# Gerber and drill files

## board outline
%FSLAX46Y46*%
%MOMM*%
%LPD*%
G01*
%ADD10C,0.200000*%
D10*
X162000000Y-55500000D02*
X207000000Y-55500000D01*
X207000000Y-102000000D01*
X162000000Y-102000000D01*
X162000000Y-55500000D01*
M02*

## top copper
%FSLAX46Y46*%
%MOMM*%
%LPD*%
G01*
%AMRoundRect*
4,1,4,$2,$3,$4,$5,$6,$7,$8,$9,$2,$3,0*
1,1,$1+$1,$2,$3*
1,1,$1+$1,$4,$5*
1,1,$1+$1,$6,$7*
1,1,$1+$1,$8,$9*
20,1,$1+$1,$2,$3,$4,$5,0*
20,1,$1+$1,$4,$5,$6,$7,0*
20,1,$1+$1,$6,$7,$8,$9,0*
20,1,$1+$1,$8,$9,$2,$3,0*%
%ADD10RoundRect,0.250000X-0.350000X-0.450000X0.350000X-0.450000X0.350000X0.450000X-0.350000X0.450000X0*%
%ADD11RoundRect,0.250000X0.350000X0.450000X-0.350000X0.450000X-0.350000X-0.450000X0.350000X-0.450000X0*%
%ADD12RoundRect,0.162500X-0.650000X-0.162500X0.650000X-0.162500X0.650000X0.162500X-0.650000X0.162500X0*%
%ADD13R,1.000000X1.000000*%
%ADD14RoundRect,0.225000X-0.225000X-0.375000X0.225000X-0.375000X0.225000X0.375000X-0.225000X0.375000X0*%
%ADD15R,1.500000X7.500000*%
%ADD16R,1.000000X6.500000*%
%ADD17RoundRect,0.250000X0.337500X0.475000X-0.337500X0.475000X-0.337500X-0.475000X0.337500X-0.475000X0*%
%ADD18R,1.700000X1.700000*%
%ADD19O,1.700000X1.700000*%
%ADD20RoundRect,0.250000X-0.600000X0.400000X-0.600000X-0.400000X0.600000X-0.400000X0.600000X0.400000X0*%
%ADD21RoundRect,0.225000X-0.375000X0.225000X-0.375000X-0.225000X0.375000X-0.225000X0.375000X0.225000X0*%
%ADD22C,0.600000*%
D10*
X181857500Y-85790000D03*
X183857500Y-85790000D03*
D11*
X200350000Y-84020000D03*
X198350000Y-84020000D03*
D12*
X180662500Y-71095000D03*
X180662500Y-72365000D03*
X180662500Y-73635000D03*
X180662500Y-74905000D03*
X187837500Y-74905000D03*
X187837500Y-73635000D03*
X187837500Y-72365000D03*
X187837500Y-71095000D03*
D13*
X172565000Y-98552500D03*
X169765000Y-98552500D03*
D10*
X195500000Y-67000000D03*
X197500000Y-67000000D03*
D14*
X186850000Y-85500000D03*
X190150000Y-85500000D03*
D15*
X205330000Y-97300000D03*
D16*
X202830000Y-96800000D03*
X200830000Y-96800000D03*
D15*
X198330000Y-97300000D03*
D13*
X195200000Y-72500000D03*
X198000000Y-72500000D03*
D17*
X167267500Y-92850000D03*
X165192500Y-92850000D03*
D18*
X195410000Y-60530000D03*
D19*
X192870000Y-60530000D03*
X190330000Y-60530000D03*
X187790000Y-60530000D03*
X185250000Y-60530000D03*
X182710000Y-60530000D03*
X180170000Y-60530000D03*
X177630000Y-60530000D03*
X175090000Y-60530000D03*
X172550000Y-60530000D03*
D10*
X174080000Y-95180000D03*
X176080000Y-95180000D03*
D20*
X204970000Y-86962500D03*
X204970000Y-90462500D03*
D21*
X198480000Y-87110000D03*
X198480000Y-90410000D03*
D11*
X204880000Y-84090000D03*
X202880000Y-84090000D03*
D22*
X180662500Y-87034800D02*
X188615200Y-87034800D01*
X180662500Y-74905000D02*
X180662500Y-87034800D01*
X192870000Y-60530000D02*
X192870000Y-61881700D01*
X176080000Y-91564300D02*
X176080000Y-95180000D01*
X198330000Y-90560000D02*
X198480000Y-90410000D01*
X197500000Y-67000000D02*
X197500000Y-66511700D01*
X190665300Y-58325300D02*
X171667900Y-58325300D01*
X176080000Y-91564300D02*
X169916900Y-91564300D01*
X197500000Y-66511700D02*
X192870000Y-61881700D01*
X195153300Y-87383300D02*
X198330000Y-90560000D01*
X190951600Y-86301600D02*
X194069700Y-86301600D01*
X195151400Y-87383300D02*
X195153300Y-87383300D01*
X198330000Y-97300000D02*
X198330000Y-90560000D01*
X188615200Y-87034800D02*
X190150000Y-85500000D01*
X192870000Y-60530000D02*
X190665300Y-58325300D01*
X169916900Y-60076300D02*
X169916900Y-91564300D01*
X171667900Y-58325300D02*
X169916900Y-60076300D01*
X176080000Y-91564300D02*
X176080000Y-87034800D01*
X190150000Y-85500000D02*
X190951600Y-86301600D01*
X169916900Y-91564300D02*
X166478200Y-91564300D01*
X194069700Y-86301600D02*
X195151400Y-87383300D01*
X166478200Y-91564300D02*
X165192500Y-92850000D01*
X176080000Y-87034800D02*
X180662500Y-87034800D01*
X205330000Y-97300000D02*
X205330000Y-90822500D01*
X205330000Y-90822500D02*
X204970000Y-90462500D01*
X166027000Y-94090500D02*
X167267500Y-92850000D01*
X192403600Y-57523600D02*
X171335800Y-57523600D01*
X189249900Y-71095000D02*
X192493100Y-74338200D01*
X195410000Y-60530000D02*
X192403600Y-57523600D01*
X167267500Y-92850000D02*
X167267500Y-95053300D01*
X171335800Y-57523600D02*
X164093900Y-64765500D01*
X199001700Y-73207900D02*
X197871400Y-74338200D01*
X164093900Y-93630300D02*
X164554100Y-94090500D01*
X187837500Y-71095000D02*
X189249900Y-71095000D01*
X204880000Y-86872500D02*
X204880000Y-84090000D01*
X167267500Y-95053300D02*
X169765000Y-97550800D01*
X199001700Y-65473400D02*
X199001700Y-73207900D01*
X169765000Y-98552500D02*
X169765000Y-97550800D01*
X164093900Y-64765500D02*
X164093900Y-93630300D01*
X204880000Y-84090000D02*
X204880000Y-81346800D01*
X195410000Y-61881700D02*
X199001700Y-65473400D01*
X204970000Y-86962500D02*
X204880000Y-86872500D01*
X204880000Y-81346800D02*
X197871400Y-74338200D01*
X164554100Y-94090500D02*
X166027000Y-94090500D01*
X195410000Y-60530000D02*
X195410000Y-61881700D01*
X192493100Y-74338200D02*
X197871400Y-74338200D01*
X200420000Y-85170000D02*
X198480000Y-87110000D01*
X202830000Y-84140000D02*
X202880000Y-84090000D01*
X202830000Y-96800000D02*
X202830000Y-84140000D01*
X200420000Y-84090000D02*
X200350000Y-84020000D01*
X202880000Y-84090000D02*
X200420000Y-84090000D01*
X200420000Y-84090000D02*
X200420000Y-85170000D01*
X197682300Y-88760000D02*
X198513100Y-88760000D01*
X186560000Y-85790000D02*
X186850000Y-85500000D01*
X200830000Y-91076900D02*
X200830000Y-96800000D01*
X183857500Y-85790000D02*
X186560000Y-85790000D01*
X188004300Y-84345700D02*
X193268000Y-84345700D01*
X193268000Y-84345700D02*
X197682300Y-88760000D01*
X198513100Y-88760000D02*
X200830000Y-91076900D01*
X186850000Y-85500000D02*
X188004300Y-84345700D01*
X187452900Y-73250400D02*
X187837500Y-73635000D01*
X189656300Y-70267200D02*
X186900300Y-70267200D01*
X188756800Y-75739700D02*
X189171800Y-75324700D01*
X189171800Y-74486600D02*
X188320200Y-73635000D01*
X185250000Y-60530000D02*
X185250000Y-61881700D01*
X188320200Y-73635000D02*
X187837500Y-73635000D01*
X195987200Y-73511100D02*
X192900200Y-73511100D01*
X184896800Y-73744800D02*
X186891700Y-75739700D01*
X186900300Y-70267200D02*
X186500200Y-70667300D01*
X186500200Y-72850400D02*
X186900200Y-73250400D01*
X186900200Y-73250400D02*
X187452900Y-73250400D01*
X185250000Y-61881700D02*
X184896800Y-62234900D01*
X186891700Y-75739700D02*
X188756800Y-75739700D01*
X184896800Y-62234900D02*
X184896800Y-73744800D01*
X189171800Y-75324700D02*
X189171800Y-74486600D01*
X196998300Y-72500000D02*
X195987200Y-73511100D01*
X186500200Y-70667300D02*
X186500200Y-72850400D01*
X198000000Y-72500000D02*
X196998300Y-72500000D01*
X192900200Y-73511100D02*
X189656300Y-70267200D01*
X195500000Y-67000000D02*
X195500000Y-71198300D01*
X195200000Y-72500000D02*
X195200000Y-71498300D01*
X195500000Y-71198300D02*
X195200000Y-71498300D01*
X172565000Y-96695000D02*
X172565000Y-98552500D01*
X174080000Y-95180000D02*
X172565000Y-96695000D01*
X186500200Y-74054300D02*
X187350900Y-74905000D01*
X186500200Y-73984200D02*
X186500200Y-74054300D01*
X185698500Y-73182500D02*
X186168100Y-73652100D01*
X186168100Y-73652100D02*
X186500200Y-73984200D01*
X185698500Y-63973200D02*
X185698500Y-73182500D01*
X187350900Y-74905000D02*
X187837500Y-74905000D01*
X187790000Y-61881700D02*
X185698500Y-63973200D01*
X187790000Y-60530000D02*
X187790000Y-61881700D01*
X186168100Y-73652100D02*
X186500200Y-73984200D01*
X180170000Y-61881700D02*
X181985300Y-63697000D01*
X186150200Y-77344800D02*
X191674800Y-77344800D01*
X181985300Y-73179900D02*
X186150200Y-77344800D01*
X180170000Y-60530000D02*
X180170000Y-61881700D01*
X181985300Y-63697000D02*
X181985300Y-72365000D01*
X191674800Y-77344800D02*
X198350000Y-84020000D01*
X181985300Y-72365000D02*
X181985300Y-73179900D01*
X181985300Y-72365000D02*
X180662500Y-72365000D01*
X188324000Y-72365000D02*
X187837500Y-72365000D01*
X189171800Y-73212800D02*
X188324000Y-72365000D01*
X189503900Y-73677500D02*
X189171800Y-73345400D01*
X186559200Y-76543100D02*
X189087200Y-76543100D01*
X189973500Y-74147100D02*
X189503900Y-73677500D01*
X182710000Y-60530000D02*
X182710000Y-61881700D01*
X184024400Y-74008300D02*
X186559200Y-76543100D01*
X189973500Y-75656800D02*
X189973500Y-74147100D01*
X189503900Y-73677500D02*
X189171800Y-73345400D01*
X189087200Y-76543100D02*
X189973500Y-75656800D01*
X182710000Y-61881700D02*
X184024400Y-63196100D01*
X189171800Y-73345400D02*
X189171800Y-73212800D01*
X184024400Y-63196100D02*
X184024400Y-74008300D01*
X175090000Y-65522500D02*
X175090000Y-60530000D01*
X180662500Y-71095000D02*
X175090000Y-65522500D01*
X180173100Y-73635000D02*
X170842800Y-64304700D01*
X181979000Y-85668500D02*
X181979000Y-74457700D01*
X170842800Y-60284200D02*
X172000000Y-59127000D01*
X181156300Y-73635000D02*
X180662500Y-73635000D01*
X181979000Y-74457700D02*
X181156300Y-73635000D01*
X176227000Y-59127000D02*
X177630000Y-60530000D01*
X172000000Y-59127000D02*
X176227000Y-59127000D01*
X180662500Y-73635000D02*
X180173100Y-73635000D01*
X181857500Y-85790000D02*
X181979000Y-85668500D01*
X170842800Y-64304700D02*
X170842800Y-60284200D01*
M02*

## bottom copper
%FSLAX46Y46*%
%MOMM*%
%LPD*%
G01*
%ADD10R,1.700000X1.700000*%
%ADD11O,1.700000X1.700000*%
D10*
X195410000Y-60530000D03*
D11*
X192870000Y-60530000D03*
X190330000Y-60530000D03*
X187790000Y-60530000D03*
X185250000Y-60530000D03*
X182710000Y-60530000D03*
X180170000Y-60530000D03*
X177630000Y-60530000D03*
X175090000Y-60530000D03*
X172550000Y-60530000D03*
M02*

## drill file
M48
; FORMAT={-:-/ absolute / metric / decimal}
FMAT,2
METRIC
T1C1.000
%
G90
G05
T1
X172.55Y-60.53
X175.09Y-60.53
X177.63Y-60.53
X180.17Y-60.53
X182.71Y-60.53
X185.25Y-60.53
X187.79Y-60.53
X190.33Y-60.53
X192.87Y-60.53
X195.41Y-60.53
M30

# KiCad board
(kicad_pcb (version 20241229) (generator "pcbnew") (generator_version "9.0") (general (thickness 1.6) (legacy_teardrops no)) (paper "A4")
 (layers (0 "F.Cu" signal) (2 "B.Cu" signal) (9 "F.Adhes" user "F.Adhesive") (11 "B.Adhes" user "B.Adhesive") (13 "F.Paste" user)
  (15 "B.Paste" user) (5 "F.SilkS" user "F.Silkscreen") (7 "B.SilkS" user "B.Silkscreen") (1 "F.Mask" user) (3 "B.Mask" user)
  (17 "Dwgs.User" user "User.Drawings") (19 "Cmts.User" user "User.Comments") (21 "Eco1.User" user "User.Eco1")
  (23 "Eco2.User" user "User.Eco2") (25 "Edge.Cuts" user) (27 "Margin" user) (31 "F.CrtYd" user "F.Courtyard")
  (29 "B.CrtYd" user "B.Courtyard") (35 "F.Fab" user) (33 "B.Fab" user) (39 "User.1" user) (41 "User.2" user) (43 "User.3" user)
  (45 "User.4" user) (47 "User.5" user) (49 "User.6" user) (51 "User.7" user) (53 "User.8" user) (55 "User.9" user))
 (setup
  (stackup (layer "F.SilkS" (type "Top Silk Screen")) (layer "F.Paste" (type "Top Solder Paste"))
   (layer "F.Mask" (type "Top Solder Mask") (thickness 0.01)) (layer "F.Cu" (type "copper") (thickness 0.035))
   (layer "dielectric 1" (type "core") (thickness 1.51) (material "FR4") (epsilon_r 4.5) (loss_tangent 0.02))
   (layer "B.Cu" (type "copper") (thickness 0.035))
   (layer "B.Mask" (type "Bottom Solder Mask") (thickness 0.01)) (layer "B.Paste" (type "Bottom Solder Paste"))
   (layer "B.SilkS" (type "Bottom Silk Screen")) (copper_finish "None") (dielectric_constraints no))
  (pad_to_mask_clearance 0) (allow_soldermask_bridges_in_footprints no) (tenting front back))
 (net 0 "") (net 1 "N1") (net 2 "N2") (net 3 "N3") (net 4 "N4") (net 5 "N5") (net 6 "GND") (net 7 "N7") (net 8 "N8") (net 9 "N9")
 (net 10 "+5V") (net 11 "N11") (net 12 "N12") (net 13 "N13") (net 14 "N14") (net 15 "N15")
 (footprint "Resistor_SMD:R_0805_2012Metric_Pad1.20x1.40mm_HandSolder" (layer "F.Cu") (at 182.8575 85.79)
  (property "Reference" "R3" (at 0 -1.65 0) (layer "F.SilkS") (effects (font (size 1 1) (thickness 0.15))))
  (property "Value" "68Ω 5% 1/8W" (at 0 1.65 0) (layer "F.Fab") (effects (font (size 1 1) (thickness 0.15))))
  (pad "1" smd roundrect (at -1 0) (size 1.2 1.4) (layers "F.Cu" "F.Mask" "F.Paste") (roundrect_rratio 0.208333) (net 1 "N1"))
  (pad "2" smd roundrect (at 1 0) (size 1.2 1.4) (layers "F.Cu" "F.Mask" "F.Paste") (roundrect_rratio 0.208333) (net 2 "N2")))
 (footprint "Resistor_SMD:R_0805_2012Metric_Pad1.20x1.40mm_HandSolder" (layer "F.Cu") (at 199.35 84.02 180)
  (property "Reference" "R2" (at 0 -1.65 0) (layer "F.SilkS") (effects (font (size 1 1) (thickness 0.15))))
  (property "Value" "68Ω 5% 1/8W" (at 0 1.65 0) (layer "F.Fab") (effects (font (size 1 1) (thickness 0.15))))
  (pad "1" smd roundrect (at -1 0 180) (size 1.2 1.4) (layers "F.Cu" "F.Mask" "F.Paste") (roundrect_rratio 0.208333) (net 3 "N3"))
  (pad "2" smd roundrect (at 1 0 180) (size 1.2 1.4) (layers "F.Cu" "F.Mask" "F.Paste") (roundrect_rratio 0.208333) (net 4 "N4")))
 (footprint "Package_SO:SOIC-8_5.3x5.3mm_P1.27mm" (layer "F.Cu") (at 184.25 73)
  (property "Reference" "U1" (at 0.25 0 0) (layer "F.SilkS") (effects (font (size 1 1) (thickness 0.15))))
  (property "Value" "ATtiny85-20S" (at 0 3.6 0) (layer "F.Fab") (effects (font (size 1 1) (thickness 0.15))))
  (pad "1" smd roundrect (at -3.5875 -1.905) (size 1.625 0.65) (layers "F.Cu" "F.Mask" "F.Paste") (roundrect_rratio 0.25) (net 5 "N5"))
  (pad "2" smd roundrect (at -3.5875 -0.635) (size 1.625 0.65) (layers "F.Cu" "F.Mask" "F.Paste") (roundrect_rratio 0.25) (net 4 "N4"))
  (pad "3" smd roundrect (at -3.5875 0.635) (size 1.625 0.65) (layers "F.Cu" "F.Mask" "F.Paste") (roundrect_rratio 0.25) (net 1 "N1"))
  (pad "4" smd roundrect (at -3.5875 1.905) (size 1.625 0.65) (layers "F.Cu" "F.Mask" "F.Paste") (roundrect_rratio 0.25) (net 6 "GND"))
  (pad "5" smd roundrect (at 3.5875 1.905) (size 1.625 0.65) (layers "F.Cu" "F.Mask" "F.Paste") (roundrect_rratio 0.25) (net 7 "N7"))
  (pad "6" smd roundrect (at 3.5875 0.635) (size 1.625 0.65) (layers "F.Cu" "F.Mask" "F.Paste") (roundrect_rratio 0.25) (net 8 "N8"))
  (pad "7" smd roundrect (at 3.5875 -0.635) (size 1.625 0.65) (layers "F.Cu" "F.Mask" "F.Paste") (roundrect_rratio 0.25) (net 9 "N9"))
  (pad "8" smd roundrect (at 3.5875 -1.905) (size 1.625 0.65) (layers "F.Cu" "F.Mask" "F.Paste") (roundrect_rratio 0.25) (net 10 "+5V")))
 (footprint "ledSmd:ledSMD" (layer "F.Cu") (at 170.765 98.5525 180)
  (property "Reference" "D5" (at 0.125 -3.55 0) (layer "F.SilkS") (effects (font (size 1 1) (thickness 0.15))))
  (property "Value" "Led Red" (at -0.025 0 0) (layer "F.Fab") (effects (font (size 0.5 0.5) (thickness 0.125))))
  (pad "1" smd rect (at -1.8 0 180) (size 1 1) (layers "F.Cu" "F.Mask" "F.Paste") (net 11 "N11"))
  (pad "2" smd rect (at 1 0 180) (size 1 1) (layers "F.Cu" "F.Mask" "F.Paste") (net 10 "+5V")))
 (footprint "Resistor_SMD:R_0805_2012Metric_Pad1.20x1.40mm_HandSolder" (layer "F.Cu") (at 196.5 67)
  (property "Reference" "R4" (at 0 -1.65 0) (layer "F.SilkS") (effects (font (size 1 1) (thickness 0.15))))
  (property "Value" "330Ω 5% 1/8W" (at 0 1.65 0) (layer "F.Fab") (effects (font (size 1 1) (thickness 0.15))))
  (pad "1" smd roundrect (at -1 0) (size 1.2 1.4) (layers "F.Cu" "F.Mask" "F.Paste") (roundrect_rratio 0.208333) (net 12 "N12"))
  (pad "2" smd roundrect (at 1 0) (size 1.2 1.4) (layers "F.Cu" "F.Mask" "F.Paste") (roundrect_rratio 0.208333) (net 6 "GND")))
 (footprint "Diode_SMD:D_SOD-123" (layer "F.Cu") (at 188.5 85.5)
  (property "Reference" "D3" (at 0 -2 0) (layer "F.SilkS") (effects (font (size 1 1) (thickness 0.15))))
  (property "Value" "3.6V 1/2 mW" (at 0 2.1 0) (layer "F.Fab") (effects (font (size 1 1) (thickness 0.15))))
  (pad "1" smd roundrect (at -1.65 0) (size 0.9 1.2) (layers "F.Cu" "F.Mask" "F.Paste") (roundrect_rratio 0.25) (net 2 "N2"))
  (pad "2" smd roundrect (at 1.65 0) (size 0.9 1.2) (layers "F.Cu" "F.Mask" "F.Paste") (roundrect_rratio 0.25) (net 6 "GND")))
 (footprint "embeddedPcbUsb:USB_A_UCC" (layer "F.Cu") (at 201.83 97.1 90)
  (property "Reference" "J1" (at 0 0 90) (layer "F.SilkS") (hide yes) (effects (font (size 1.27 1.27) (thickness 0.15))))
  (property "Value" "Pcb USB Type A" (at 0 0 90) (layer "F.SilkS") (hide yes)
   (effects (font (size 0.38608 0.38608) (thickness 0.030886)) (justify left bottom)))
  (pad "1" smd rect (at -0.2 3.5 90) (size 7.5 1.5) (layers "F.Cu" "F.Mask" "F.Paste") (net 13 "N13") (solder_mask_margin 0.1016))
  (pad "2" smd rect (at 0.3 1 90) (size 6.5 1) (layers "F.Cu" "F.Mask" "F.Paste") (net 3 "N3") (solder_mask_margin 0.1016))
  (pad "3" smd rect (at 0.3 -1 90) (size 6.5 1) (layers "F.Cu" "F.Mask" "F.Paste") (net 2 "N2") (solder_mask_margin 0.1016))
  (pad "4" smd rect (at -0.2 -3.5 90) (size 7.5 1.5) (layers "F.Cu" "F.Mask" "F.Paste") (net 6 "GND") (solder_mask_margin 0.1016)))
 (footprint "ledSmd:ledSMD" (layer "F.Cu") (at 197 72.5)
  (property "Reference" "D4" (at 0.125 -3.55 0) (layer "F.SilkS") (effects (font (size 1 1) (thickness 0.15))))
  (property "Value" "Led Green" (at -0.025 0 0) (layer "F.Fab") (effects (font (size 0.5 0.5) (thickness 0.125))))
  (pad "1" smd rect (at -1.8 0) (size 1 1) (layers "F.Cu" "F.Mask" "F.Paste") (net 12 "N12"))
  (pad "2" smd rect (at 1 0) (size 1 1) (layers "F.Cu" "F.Mask" "F.Paste") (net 8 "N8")))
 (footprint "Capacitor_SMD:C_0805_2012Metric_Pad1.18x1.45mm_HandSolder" (layer "F.Cu") (at 166.23 92.85 180)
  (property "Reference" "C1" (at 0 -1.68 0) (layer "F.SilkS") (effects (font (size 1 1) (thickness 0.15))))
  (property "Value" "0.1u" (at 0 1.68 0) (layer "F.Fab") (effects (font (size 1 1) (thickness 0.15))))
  (pad "1" smd roundrect (at -1.0375 0 180) (size 1.175 1.45) (layers "F.Cu" "F.Mask" "F.Paste") (roundrect_rratio 0.212766) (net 10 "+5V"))
  (pad "2" smd roundrect (at 1.0375 0 180) (size 1.175 1.45) (layers "F.Cu" "F.Mask" "F.Paste") (roundrect_rratio 0.212766) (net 6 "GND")))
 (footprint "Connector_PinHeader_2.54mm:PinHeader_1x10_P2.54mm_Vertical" (layer "F.Cu") (at 195.41 60.53 -90)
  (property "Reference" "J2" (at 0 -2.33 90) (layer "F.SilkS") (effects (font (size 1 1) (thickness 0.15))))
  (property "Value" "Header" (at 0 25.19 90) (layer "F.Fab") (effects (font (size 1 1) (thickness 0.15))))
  (pad "1" thru_hole rect (at 0 0 270) (size 1.7 1.7) (drill 1) (layers "*.Cu" "*.Mask") (remove_unused_layers no) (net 10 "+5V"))
  (pad "2" thru_hole oval (at 0 2.54 270) (size 1.7 1.7) (drill 1) (layers "*.Cu" "*.Mask") (remove_unused_layers no) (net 6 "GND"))
  (pad "3" thru_hole oval (at 0 5.08 270) (size 1.7 1.7) (drill 1) (layers "*.Cu" "*.Mask") (remove_unused_layers no) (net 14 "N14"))
  (pad "4" thru_hole oval (at 0 7.62 270) (size 1.7 1.7) (drill 1) (layers "*.Cu" "*.Mask") (remove_unused_layers no) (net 7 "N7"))
  (pad "5" thru_hole oval (at 0 10.16 270) (size 1.7 1.7) (drill 1) (layers "*.Cu" "*.Mask") (remove_unused_layers no) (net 8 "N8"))
  (pad "6" thru_hole oval (at 0 12.7 270) (size 1.7 1.7) (drill 1) (layers "*.Cu" "*.Mask") (remove_unused_layers no) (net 9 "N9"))
  (pad "7" thru_hole oval (at 0 15.24 270) (size 1.7 1.7) (drill 1) (layers "*.Cu" "*.Mask") (remove_unused_layers no) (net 4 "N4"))
  (pad "8" thru_hole oval (at 0 17.78 270) (size 1.7 1.7) (drill 1) (layers "*.Cu" "*.Mask") (remove_unused_layers no) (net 1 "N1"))
  (pad "9" thru_hole oval (at 0 20.32 270) (size 1.7 1.7) (drill 1) (layers "*.Cu" "*.Mask") (remove_unused_layers no) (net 5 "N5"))
  (pad "10" thru_hole oval (at 0 22.86 270) (size 1.7 1.7) (drill 1) (layers "*.Cu" "*.Mask") (remove_unused_layers no) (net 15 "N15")))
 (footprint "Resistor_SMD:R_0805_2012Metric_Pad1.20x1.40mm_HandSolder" (layer "F.Cu") (at 175.08 95.18)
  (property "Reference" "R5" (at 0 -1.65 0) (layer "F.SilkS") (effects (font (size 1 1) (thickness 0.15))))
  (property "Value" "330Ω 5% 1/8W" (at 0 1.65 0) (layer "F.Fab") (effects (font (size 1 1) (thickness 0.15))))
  (pad "1" smd roundrect (at -1 0) (size 1.2 1.4) (layers "F.Cu" "F.Mask" "F.Paste") (roundrect_rratio 0.208333) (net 11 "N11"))
  (pad "2" smd roundrect (at 1 0) (size 1.2 1.4) (layers "F.Cu" "F.Mask" "F.Paste") (roundrect_rratio 0.208333) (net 6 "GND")))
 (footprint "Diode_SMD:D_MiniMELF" (layer "F.Cu") (at 204.97 88.7125 -90)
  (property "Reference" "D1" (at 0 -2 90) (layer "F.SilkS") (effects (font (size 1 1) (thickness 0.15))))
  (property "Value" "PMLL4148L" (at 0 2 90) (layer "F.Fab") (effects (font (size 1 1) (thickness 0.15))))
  (pad "1" smd roundrect (at -1.75 0 270) (size 1.3 1.7) (layers "F.Cu" "F.Mask" "F.Paste") (roundrect_rratio 0.1923076923) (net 10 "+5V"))
  (pad "2" smd roundrect (at 1.75 0 270) (size 1.3 1.7) (layers "F.Cu" "F.Mask" "F.Paste") (roundrect_rratio 0.1923076923) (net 13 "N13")))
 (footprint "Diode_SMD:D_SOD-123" (layer "F.Cu") (at 198.48 88.76 -90)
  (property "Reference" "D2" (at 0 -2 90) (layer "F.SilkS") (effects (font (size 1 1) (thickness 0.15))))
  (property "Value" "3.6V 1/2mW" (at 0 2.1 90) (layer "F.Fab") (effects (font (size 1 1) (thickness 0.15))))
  (pad "1" smd roundrect (at -1.65 0 270) (size 0.9 1.2) (layers "F.Cu" "F.Mask" "F.Paste") (roundrect_rratio 0.25) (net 3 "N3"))
  (pad "2" smd roundrect (at 1.65 0 270) (size 0.9 1.2) (layers "F.Cu" "F.Mask" "F.Paste") (roundrect_rratio 0.25) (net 6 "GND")))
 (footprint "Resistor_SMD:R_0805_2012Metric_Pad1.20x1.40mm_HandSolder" (layer "F.Cu") (at 203.88 84.09 180)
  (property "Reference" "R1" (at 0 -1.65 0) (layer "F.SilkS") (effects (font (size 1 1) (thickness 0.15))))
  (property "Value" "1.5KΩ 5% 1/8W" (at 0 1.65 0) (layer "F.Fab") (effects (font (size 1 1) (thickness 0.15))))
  (pad "1" smd roundrect (at -1 0 180) (size 1.2 1.4) (layers "F.Cu" "F.Mask" "F.Paste") (roundrect_rratio 0.208333) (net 10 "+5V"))
  (pad "2" smd roundrect (at 1 0 180) (size 1.2 1.4) (layers "F.Cu" "F.Mask" "F.Paste") (roundrect_rratio 0.208333) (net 3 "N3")))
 (gr_rect (start 162 55.5) (end 207 102) (stroke (width 0.2) (type solid)) (fill no) (layer "Edge.Cuts"))
 (segment (start 180.6625 87.0348) (end 188.6152 87.0348) (width 0.6) (layer "F.Cu") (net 6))
 (segment (start 180.6625 74.905) (end 180.6625 87.0348) (width 0.6) (layer "F.Cu") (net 6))
 (segment (start 192.87 60.53) (end 192.87 61.8817) (width 0.6) (layer "F.Cu") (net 6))
 (segment (start 176.08 91.5643) (end 176.08 95.18) (width 0.6) (layer "F.Cu") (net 6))
 (segment (start 198.33 90.56) (end 198.48 90.41) (width 0.6) (layer "F.Cu") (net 6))
 (segment (start 197.5 67) (end 197.5 66.5117) (width 0.6) (layer "F.Cu") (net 6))
 (segment (start 190.6653 58.3253) (end 171.6679 58.3253) (width 0.6) (layer "F.Cu") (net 6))
 (segment (start 176.08 91.5643) (end 169.9169 91.5643) (width 0.6) (layer "F.Cu") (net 6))
 (segment (start 197.5 66.5117) (end 192.87 61.8817) (width 0.6) (layer "F.Cu") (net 6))
 (segment (start 195.1533 87.3833) (end 198.33 90.56) (width 0.6) (layer "F.Cu") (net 6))
 (segment (start 190.9516 86.3016) (end 194.0697 86.3016) (width 0.6) (layer "F.Cu") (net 6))
 (segment (start 195.1514 87.3833) (end 195.1533 87.3833) (width 0.6) (layer "F.Cu") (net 6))
 (segment (start 198.33 97.3) (end 198.33 90.56) (width 0.6) (layer "F.Cu") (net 6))
 (segment (start 188.6152 87.0348) (end 190.15 85.5) (width 0.6) (layer "F.Cu") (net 6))
 (segment (start 192.87 60.53) (end 190.6653 58.3253) (width 0.6) (layer "F.Cu") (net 6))
 (segment (start 169.9169 60.0763) (end 169.9169 91.5643) (width 0.6) (layer "F.Cu") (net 6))
 (segment (start 171.6679 58.3253) (end 169.9169 60.0763) (width 0.6) (layer "F.Cu") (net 6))
 (segment (start 176.08 91.5643) (end 176.08 87.0348) (width 0.6) (layer "F.Cu") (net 6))
 (segment (start 190.15 85.5) (end 190.9516 86.3016) (width 0.6) (layer "F.Cu") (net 6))
 (segment (start 169.9169 91.5643) (end 166.4782 91.5643) (width 0.6) (layer "F.Cu") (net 6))
 (segment (start 194.0697 86.3016) (end 195.1514 87.3833) (width 0.6) (layer "F.Cu") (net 6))
 (segment (start 166.4782 91.5643) (end 165.1925 92.85) (width 0.6) (layer "F.Cu") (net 6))
 (segment (start 176.08 87.0348) (end 180.6625 87.0348) (width 0.6) (layer "F.Cu") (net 6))
 (segment (start 205.33 97.3) (end 205.33 90.8225) (width 0.6) (layer "F.Cu") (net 13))
 (segment (start 205.33 90.8225) (end 204.97 90.4625) (width 0.6) (layer "F.Cu") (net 13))
 (segment (start 166.027 94.0905) (end 167.2675 92.85) (width 0.6) (layer "F.Cu") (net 10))
 (segment (start 192.4036 57.5236) (end 171.3358 57.5236) (width 0.6) (layer "F.Cu") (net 10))
 (segment (start 189.2499 71.095) (end 192.4931 74.3382) (width 0.6) (layer "F.Cu") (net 10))
 (segment (start 195.41 60.53) (end 192.4036 57.5236) (width 0.6) (layer "F.Cu") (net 10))
 (segment (start 167.2675 92.85) (end 167.2675 95.0533) (width 0.6) (layer "F.Cu") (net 10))
 (segment (start 171.3358 57.5236) (end 164.0939 64.7655) (width 0.6) (layer "F.Cu") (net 10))
 (segment (start 199.0017 73.2079) (end 197.8714 74.3382) (width 0.6) (layer "F.Cu") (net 10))
 (segment (start 164.0939 93.6303) (end 164.5541 94.0905) (width 0.6) (layer "F.Cu") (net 10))
 (segment (start 187.8375 71.095) (end 189.2499 71.095) (width 0.6) (layer "F.Cu") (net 10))
 (segment (start 204.88 86.8725) (end 204.88 84.09) (width 0.6) (layer "F.Cu") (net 10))
 (segment (start 167.2675 95.0533) (end 169.765 97.5508) (width 0.6) (layer "F.Cu") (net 10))
 (segment (start 199.0017 65.4734) (end 199.0017 73.2079) (width 0.6) (layer "F.Cu") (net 10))
 (segment (start 169.765 98.5525) (end 169.765 97.5508) (width 0.6) (layer "F.Cu") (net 10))
 (segment (start 164.0939 64.7655) (end 164.0939 93.6303) (width 0.6) (layer "F.Cu") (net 10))
 (segment (start 204.88 84.09) (end 204.88 81.3468) (width 0.6) (layer "F.Cu") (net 10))
 (segment (start 195.41 61.8817) (end 199.0017 65.4734) (width 0.6) (layer "F.Cu") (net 10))
 (segment (start 204.97 86.9625) (end 204.88 86.8725) (width 0.6) (layer "F.Cu") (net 10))
 (segment (start 204.88 81.3468) (end 197.8714 74.3382) (width 0.6) (layer "F.Cu") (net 10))
 (segment (start 164.5541 94.0905) (end 166.027 94.0905) (width 0.6) (layer "F.Cu") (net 10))
 (segment (start 195.41 60.53) (end 195.41 61.8817) (width 0.6) (layer "F.Cu") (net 10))
 (segment (start 192.4931 74.3382) (end 197.8714 74.3382) (width 0.6) (layer "F.Cu") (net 10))
 (segment (start 200.42 85.17) (end 198.48 87.11) (width 0.6) (layer "F.Cu") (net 3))
 (segment (start 202.83 84.14) (end 202.88 84.09) (width 0.6) (layer "F.Cu") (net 3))
 (segment (start 202.83 96.8) (end 202.83 84.14) (width 0.6) (layer "F.Cu") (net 3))
 (segment (start 200.42 84.09) (end 200.35 84.02) (width 0.6) (layer "F.Cu") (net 3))
 (segment (start 202.88 84.09) (end 200.42 84.09) (width 0.6) (layer "F.Cu") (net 3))
 (segment (start 200.42 84.09) (end 200.42 85.17) (width 0.6) (layer "F.Cu") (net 3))
 (segment (start 197.6823 88.76) (end 198.5131 88.76) (width 0.6) (layer "F.Cu") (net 2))
 (segment (start 186.56 85.79) (end 186.85 85.5) (width 0.6) (layer "F.Cu") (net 2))
 (segment (start 200.83 91.0769) (end 200.83 96.8) (width 0.6) (layer "F.Cu") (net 2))
 (segment (start 183.8575 85.79) (end 186.56 85.79) (width 0.6) (layer "F.Cu") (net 2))
 (segment (start 188.0043 84.3457) (end 193.268 84.3457) (width 0.6) (layer "F.Cu") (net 2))
 (segment (start 193.268 84.3457) (end 197.6823 88.76) (width 0.6) (layer "F.Cu") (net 2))
 (segment (start 198.5131 88.76) (end 200.83 91.0769) (width 0.6) (layer "F.Cu") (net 2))
 (segment (start 186.85 85.5) (end 188.0043 84.3457) (width 0.6) (layer "F.Cu") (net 2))
 (segment (start 187.4529 73.2504) (end 187.8375 73.635) (width 0.6) (layer "F.Cu") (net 8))
 (segment (start 189.6563 70.2672) (end 186.9003 70.2672) (width 0.6) (layer "F.Cu") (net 8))
 (segment (start 188.7568 75.7397) (end 189.1718 75.3247) (width 0.6) (layer "F.Cu") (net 8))
 (segment (start 189.1718 74.4866) (end 188.3202 73.635) (width 0.6) (layer "F.Cu") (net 8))
 (segment (start 185.25 60.53) (end 185.25 61.8817) (width 0.6) (layer "F.Cu") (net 8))
 (segment (start 188.3202 73.635) (end 187.8375 73.635) (width 0.6) (layer "F.Cu") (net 8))
 (segment (start 195.9872 73.5111) (end 192.9002 73.5111) (width 0.6) (layer "F.Cu") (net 8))
 (segment (start 184.8968 73.7448) (end 186.8917 75.7397) (width 0.6) (layer "F.Cu") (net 8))
 (segment (start 186.9003 70.2672) (end 186.5002 70.6673) (width 0.6) (layer "F.Cu") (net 8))
 (segment (start 186.5002 72.8504) (end 186.9002 73.2504) (width 0.6) (layer "F.Cu") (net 8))
 (segment (start 186.9002 73.2504) (end 187.4529 73.2504) (width 0.6) (layer "F.Cu") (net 8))
 (segment (start 185.25 61.8817) (end 184.8968 62.2349) (width 0.6) (layer "F.Cu") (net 8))
 (segment (start 186.8917 75.7397) (end 188.7568 75.7397) (width 0.6) (layer "F.Cu") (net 8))
 (segment (start 184.8968 62.2349) (end 184.8968 73.7448) (width 0.6) (layer "F.Cu") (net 8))
 (segment (start 189.1718 75.3247) (end 189.1718 74.4866) (width 0.6) (layer "F.Cu") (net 8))
 (segment (start 196.9983 72.5) (end 195.9872 73.5111) (width 0.6) (layer "F.Cu") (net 8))
 (segment (start 186.5002 70.6673) (end 186.5002 72.8504) (width 0.6) (layer "F.Cu") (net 8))
 (segment (start 198 72.5) (end 196.9983 72.5) (width 0.6) (layer "F.Cu") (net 8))
 (segment (start 192.9002 73.5111) (end 189.6563 70.2672) (width 0.6) (layer "F.Cu") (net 8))
 (segment (start 195.5 67) (end 195.5 71.1983) (width 0.6) (layer "F.Cu") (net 12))
 (segment (start 195.2 72.5) (end 195.2 71.4983) (width 0.6) (layer "F.Cu") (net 12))
 (segment (start 195.5 71.1983) (end 195.2 71.4983) (width 0.6) (layer "F.Cu") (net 12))
 (segment (start 172.565 96.695) (end 172.565 98.5525) (width 0.6) (layer "F.Cu") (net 11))
 (segment (start 174.08 95.18) (end 172.565 96.695) (width 0.6) (layer "F.Cu") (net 11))
 (segment (start 186.5002 74.0543) (end 187.3509 74.905) (width 0.6) (layer "F.Cu") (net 7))
 (segment (start 186.5002 73.9842) (end 186.5002 74.0543) (width 0.6) (layer "F.Cu") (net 7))
 (segment (start 185.6985 73.1825) (end 186.1681 73.6521) (width 0.6) (layer "F.Cu") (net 7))
 (segment (start 186.1681 73.6521) (end 186.5002 73.9842) (width 0.6) (layer "F.Cu") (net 7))
 (segment (start 185.6985 63.9732) (end 185.6985 73.1825) (width 0.6) (layer "F.Cu") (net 7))
 (segment (start 187.3509 74.905) (end 187.8375 74.905) (width 0.6) (layer "F.Cu") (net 7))
 (segment (start 187.79 61.8817) (end 185.6985 63.9732) (width 0.6) (layer "F.Cu") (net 7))
 (segment (start 187.79 60.53) (end 187.79 61.8817) (width 0.6) (layer "F.Cu") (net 7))
 (segment (start 186.1681 73.6521) (end 186.5002 73.9842) (width 0.6) (layer "F.Cu") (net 7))
 (segment (start 180.17 61.8817) (end 181.9853 63.697) (width 0.6) (layer "F.Cu") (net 4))
 (segment (start 186.1502 77.3448) (end 191.6748 77.3448) (width 0.6) (layer "F.Cu") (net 4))
 (segment (start 181.9853 73.1799) (end 186.1502 77.3448) (width 0.6) (layer "F.Cu") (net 4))
 (segment (start 180.17 60.53) (end 180.17 61.8817) (width 0.6) (layer "F.Cu") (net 4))
 (segment (start 181.9853 63.697) (end 181.9853 72.365) (width 0.6) (layer "F.Cu") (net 4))
 (segment (start 191.6748 77.3448) (end 198.35 84.02) (width 0.6) (layer "F.Cu") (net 4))
 (segment (start 181.9853 72.365) (end 181.9853 73.1799) (width 0.6) (layer "F.Cu") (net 4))
 (segment (start 181.9853 72.365) (end 180.6625 72.365) (width 0.6) (layer "F.Cu") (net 4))
 (segment (start 188.324 72.365) (end 187.8375 72.365) (width 0.6) (layer "F.Cu") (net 9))
 (segment (start 189.1718 73.2128) (end 188.324 72.365) (width 0.6) (layer "F.Cu") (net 9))
 (segment (start 189.5039 73.6775) (end 189.1718 73.3454) (width 0.6) (layer "F.Cu") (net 9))
 (segment (start 186.5592 76.5431) (end 189.0872 76.5431) (width 0.6) (layer "F.Cu") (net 9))
 (segment (start 189.9735 74.1471) (end 189.5039 73.6775) (width 0.6) (layer "F.Cu") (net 9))
 (segment (start 182.71 60.53) (end 182.71 61.8817) (width 0.6) (layer "F.Cu") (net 9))
 (segment (start 184.0244 74.0083) (end 186.5592 76.5431) (width 0.6) (layer "F.Cu") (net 9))
 (segment (start 189.9735 75.6568) (end 189.9735 74.1471) (width 0.6) (layer "F.Cu") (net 9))
 (segment (start 189.5039 73.6775) (end 189.1718 73.3454) (width 0.6) (layer "F.Cu") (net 9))
 (segment (start 189.0872 76.5431) (end 189.9735 75.6568) (width 0.6) (layer "F.Cu") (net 9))
 (segment (start 182.71 61.8817) (end 184.0244 63.1961) (width 0.6) (layer "F.Cu") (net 9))
 (segment (start 189.1718 73.3454) (end 189.1718 73.2128) (width 0.6) (layer "F.Cu") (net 9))
 (segment (start 184.0244 63.1961) (end 184.0244 74.0083) (width 0.6) (layer "F.Cu") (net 9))
 (segment (start 175.09 65.5225) (end 175.09 60.53) (width 0.6) (layer "F.Cu") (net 5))
 (segment (start 180.6625 71.095) (end 175.09 65.5225) (width 0.6) (layer "F.Cu") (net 5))
 (segment (start 180.1731 73.635) (end 170.8428 64.3047) (width 0.6) (layer "F.Cu") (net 1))
 (segment (start 181.979 85.6685) (end 181.979 74.4577) (width 0.6) (layer "F.Cu") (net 1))
 (segment (start 170.8428 60.2842) (end 172 59.127) (width 0.6) (layer "F.Cu") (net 1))
 (segment (start 181.1563 73.635) (end 180.6625 73.635) (width 0.6) (layer "F.Cu") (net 1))
 (segment (start 181.979 74.4577) (end 181.1563 73.635) (width 0.6) (layer "F.Cu") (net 1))
 (segment (start 176.227 59.127) (end 177.63 60.53) (width 0.6) (layer "F.Cu") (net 1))
 (segment (start 172 59.127) (end 176.227 59.127) (width 0.6) (layer "F.Cu") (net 1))
 (segment (start 180.6625 73.635) (end 180.1731 73.635) (width 0.6) (layer "F.Cu") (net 1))
 (segment (start 181.8575 85.79) (end 181.979 85.6685) (width 0.6) (layer "F.Cu") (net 1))
 (segment (start 170.8428 64.3047) (end 170.8428 60.2842) (width 0.6) (layer "F.Cu") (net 1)))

